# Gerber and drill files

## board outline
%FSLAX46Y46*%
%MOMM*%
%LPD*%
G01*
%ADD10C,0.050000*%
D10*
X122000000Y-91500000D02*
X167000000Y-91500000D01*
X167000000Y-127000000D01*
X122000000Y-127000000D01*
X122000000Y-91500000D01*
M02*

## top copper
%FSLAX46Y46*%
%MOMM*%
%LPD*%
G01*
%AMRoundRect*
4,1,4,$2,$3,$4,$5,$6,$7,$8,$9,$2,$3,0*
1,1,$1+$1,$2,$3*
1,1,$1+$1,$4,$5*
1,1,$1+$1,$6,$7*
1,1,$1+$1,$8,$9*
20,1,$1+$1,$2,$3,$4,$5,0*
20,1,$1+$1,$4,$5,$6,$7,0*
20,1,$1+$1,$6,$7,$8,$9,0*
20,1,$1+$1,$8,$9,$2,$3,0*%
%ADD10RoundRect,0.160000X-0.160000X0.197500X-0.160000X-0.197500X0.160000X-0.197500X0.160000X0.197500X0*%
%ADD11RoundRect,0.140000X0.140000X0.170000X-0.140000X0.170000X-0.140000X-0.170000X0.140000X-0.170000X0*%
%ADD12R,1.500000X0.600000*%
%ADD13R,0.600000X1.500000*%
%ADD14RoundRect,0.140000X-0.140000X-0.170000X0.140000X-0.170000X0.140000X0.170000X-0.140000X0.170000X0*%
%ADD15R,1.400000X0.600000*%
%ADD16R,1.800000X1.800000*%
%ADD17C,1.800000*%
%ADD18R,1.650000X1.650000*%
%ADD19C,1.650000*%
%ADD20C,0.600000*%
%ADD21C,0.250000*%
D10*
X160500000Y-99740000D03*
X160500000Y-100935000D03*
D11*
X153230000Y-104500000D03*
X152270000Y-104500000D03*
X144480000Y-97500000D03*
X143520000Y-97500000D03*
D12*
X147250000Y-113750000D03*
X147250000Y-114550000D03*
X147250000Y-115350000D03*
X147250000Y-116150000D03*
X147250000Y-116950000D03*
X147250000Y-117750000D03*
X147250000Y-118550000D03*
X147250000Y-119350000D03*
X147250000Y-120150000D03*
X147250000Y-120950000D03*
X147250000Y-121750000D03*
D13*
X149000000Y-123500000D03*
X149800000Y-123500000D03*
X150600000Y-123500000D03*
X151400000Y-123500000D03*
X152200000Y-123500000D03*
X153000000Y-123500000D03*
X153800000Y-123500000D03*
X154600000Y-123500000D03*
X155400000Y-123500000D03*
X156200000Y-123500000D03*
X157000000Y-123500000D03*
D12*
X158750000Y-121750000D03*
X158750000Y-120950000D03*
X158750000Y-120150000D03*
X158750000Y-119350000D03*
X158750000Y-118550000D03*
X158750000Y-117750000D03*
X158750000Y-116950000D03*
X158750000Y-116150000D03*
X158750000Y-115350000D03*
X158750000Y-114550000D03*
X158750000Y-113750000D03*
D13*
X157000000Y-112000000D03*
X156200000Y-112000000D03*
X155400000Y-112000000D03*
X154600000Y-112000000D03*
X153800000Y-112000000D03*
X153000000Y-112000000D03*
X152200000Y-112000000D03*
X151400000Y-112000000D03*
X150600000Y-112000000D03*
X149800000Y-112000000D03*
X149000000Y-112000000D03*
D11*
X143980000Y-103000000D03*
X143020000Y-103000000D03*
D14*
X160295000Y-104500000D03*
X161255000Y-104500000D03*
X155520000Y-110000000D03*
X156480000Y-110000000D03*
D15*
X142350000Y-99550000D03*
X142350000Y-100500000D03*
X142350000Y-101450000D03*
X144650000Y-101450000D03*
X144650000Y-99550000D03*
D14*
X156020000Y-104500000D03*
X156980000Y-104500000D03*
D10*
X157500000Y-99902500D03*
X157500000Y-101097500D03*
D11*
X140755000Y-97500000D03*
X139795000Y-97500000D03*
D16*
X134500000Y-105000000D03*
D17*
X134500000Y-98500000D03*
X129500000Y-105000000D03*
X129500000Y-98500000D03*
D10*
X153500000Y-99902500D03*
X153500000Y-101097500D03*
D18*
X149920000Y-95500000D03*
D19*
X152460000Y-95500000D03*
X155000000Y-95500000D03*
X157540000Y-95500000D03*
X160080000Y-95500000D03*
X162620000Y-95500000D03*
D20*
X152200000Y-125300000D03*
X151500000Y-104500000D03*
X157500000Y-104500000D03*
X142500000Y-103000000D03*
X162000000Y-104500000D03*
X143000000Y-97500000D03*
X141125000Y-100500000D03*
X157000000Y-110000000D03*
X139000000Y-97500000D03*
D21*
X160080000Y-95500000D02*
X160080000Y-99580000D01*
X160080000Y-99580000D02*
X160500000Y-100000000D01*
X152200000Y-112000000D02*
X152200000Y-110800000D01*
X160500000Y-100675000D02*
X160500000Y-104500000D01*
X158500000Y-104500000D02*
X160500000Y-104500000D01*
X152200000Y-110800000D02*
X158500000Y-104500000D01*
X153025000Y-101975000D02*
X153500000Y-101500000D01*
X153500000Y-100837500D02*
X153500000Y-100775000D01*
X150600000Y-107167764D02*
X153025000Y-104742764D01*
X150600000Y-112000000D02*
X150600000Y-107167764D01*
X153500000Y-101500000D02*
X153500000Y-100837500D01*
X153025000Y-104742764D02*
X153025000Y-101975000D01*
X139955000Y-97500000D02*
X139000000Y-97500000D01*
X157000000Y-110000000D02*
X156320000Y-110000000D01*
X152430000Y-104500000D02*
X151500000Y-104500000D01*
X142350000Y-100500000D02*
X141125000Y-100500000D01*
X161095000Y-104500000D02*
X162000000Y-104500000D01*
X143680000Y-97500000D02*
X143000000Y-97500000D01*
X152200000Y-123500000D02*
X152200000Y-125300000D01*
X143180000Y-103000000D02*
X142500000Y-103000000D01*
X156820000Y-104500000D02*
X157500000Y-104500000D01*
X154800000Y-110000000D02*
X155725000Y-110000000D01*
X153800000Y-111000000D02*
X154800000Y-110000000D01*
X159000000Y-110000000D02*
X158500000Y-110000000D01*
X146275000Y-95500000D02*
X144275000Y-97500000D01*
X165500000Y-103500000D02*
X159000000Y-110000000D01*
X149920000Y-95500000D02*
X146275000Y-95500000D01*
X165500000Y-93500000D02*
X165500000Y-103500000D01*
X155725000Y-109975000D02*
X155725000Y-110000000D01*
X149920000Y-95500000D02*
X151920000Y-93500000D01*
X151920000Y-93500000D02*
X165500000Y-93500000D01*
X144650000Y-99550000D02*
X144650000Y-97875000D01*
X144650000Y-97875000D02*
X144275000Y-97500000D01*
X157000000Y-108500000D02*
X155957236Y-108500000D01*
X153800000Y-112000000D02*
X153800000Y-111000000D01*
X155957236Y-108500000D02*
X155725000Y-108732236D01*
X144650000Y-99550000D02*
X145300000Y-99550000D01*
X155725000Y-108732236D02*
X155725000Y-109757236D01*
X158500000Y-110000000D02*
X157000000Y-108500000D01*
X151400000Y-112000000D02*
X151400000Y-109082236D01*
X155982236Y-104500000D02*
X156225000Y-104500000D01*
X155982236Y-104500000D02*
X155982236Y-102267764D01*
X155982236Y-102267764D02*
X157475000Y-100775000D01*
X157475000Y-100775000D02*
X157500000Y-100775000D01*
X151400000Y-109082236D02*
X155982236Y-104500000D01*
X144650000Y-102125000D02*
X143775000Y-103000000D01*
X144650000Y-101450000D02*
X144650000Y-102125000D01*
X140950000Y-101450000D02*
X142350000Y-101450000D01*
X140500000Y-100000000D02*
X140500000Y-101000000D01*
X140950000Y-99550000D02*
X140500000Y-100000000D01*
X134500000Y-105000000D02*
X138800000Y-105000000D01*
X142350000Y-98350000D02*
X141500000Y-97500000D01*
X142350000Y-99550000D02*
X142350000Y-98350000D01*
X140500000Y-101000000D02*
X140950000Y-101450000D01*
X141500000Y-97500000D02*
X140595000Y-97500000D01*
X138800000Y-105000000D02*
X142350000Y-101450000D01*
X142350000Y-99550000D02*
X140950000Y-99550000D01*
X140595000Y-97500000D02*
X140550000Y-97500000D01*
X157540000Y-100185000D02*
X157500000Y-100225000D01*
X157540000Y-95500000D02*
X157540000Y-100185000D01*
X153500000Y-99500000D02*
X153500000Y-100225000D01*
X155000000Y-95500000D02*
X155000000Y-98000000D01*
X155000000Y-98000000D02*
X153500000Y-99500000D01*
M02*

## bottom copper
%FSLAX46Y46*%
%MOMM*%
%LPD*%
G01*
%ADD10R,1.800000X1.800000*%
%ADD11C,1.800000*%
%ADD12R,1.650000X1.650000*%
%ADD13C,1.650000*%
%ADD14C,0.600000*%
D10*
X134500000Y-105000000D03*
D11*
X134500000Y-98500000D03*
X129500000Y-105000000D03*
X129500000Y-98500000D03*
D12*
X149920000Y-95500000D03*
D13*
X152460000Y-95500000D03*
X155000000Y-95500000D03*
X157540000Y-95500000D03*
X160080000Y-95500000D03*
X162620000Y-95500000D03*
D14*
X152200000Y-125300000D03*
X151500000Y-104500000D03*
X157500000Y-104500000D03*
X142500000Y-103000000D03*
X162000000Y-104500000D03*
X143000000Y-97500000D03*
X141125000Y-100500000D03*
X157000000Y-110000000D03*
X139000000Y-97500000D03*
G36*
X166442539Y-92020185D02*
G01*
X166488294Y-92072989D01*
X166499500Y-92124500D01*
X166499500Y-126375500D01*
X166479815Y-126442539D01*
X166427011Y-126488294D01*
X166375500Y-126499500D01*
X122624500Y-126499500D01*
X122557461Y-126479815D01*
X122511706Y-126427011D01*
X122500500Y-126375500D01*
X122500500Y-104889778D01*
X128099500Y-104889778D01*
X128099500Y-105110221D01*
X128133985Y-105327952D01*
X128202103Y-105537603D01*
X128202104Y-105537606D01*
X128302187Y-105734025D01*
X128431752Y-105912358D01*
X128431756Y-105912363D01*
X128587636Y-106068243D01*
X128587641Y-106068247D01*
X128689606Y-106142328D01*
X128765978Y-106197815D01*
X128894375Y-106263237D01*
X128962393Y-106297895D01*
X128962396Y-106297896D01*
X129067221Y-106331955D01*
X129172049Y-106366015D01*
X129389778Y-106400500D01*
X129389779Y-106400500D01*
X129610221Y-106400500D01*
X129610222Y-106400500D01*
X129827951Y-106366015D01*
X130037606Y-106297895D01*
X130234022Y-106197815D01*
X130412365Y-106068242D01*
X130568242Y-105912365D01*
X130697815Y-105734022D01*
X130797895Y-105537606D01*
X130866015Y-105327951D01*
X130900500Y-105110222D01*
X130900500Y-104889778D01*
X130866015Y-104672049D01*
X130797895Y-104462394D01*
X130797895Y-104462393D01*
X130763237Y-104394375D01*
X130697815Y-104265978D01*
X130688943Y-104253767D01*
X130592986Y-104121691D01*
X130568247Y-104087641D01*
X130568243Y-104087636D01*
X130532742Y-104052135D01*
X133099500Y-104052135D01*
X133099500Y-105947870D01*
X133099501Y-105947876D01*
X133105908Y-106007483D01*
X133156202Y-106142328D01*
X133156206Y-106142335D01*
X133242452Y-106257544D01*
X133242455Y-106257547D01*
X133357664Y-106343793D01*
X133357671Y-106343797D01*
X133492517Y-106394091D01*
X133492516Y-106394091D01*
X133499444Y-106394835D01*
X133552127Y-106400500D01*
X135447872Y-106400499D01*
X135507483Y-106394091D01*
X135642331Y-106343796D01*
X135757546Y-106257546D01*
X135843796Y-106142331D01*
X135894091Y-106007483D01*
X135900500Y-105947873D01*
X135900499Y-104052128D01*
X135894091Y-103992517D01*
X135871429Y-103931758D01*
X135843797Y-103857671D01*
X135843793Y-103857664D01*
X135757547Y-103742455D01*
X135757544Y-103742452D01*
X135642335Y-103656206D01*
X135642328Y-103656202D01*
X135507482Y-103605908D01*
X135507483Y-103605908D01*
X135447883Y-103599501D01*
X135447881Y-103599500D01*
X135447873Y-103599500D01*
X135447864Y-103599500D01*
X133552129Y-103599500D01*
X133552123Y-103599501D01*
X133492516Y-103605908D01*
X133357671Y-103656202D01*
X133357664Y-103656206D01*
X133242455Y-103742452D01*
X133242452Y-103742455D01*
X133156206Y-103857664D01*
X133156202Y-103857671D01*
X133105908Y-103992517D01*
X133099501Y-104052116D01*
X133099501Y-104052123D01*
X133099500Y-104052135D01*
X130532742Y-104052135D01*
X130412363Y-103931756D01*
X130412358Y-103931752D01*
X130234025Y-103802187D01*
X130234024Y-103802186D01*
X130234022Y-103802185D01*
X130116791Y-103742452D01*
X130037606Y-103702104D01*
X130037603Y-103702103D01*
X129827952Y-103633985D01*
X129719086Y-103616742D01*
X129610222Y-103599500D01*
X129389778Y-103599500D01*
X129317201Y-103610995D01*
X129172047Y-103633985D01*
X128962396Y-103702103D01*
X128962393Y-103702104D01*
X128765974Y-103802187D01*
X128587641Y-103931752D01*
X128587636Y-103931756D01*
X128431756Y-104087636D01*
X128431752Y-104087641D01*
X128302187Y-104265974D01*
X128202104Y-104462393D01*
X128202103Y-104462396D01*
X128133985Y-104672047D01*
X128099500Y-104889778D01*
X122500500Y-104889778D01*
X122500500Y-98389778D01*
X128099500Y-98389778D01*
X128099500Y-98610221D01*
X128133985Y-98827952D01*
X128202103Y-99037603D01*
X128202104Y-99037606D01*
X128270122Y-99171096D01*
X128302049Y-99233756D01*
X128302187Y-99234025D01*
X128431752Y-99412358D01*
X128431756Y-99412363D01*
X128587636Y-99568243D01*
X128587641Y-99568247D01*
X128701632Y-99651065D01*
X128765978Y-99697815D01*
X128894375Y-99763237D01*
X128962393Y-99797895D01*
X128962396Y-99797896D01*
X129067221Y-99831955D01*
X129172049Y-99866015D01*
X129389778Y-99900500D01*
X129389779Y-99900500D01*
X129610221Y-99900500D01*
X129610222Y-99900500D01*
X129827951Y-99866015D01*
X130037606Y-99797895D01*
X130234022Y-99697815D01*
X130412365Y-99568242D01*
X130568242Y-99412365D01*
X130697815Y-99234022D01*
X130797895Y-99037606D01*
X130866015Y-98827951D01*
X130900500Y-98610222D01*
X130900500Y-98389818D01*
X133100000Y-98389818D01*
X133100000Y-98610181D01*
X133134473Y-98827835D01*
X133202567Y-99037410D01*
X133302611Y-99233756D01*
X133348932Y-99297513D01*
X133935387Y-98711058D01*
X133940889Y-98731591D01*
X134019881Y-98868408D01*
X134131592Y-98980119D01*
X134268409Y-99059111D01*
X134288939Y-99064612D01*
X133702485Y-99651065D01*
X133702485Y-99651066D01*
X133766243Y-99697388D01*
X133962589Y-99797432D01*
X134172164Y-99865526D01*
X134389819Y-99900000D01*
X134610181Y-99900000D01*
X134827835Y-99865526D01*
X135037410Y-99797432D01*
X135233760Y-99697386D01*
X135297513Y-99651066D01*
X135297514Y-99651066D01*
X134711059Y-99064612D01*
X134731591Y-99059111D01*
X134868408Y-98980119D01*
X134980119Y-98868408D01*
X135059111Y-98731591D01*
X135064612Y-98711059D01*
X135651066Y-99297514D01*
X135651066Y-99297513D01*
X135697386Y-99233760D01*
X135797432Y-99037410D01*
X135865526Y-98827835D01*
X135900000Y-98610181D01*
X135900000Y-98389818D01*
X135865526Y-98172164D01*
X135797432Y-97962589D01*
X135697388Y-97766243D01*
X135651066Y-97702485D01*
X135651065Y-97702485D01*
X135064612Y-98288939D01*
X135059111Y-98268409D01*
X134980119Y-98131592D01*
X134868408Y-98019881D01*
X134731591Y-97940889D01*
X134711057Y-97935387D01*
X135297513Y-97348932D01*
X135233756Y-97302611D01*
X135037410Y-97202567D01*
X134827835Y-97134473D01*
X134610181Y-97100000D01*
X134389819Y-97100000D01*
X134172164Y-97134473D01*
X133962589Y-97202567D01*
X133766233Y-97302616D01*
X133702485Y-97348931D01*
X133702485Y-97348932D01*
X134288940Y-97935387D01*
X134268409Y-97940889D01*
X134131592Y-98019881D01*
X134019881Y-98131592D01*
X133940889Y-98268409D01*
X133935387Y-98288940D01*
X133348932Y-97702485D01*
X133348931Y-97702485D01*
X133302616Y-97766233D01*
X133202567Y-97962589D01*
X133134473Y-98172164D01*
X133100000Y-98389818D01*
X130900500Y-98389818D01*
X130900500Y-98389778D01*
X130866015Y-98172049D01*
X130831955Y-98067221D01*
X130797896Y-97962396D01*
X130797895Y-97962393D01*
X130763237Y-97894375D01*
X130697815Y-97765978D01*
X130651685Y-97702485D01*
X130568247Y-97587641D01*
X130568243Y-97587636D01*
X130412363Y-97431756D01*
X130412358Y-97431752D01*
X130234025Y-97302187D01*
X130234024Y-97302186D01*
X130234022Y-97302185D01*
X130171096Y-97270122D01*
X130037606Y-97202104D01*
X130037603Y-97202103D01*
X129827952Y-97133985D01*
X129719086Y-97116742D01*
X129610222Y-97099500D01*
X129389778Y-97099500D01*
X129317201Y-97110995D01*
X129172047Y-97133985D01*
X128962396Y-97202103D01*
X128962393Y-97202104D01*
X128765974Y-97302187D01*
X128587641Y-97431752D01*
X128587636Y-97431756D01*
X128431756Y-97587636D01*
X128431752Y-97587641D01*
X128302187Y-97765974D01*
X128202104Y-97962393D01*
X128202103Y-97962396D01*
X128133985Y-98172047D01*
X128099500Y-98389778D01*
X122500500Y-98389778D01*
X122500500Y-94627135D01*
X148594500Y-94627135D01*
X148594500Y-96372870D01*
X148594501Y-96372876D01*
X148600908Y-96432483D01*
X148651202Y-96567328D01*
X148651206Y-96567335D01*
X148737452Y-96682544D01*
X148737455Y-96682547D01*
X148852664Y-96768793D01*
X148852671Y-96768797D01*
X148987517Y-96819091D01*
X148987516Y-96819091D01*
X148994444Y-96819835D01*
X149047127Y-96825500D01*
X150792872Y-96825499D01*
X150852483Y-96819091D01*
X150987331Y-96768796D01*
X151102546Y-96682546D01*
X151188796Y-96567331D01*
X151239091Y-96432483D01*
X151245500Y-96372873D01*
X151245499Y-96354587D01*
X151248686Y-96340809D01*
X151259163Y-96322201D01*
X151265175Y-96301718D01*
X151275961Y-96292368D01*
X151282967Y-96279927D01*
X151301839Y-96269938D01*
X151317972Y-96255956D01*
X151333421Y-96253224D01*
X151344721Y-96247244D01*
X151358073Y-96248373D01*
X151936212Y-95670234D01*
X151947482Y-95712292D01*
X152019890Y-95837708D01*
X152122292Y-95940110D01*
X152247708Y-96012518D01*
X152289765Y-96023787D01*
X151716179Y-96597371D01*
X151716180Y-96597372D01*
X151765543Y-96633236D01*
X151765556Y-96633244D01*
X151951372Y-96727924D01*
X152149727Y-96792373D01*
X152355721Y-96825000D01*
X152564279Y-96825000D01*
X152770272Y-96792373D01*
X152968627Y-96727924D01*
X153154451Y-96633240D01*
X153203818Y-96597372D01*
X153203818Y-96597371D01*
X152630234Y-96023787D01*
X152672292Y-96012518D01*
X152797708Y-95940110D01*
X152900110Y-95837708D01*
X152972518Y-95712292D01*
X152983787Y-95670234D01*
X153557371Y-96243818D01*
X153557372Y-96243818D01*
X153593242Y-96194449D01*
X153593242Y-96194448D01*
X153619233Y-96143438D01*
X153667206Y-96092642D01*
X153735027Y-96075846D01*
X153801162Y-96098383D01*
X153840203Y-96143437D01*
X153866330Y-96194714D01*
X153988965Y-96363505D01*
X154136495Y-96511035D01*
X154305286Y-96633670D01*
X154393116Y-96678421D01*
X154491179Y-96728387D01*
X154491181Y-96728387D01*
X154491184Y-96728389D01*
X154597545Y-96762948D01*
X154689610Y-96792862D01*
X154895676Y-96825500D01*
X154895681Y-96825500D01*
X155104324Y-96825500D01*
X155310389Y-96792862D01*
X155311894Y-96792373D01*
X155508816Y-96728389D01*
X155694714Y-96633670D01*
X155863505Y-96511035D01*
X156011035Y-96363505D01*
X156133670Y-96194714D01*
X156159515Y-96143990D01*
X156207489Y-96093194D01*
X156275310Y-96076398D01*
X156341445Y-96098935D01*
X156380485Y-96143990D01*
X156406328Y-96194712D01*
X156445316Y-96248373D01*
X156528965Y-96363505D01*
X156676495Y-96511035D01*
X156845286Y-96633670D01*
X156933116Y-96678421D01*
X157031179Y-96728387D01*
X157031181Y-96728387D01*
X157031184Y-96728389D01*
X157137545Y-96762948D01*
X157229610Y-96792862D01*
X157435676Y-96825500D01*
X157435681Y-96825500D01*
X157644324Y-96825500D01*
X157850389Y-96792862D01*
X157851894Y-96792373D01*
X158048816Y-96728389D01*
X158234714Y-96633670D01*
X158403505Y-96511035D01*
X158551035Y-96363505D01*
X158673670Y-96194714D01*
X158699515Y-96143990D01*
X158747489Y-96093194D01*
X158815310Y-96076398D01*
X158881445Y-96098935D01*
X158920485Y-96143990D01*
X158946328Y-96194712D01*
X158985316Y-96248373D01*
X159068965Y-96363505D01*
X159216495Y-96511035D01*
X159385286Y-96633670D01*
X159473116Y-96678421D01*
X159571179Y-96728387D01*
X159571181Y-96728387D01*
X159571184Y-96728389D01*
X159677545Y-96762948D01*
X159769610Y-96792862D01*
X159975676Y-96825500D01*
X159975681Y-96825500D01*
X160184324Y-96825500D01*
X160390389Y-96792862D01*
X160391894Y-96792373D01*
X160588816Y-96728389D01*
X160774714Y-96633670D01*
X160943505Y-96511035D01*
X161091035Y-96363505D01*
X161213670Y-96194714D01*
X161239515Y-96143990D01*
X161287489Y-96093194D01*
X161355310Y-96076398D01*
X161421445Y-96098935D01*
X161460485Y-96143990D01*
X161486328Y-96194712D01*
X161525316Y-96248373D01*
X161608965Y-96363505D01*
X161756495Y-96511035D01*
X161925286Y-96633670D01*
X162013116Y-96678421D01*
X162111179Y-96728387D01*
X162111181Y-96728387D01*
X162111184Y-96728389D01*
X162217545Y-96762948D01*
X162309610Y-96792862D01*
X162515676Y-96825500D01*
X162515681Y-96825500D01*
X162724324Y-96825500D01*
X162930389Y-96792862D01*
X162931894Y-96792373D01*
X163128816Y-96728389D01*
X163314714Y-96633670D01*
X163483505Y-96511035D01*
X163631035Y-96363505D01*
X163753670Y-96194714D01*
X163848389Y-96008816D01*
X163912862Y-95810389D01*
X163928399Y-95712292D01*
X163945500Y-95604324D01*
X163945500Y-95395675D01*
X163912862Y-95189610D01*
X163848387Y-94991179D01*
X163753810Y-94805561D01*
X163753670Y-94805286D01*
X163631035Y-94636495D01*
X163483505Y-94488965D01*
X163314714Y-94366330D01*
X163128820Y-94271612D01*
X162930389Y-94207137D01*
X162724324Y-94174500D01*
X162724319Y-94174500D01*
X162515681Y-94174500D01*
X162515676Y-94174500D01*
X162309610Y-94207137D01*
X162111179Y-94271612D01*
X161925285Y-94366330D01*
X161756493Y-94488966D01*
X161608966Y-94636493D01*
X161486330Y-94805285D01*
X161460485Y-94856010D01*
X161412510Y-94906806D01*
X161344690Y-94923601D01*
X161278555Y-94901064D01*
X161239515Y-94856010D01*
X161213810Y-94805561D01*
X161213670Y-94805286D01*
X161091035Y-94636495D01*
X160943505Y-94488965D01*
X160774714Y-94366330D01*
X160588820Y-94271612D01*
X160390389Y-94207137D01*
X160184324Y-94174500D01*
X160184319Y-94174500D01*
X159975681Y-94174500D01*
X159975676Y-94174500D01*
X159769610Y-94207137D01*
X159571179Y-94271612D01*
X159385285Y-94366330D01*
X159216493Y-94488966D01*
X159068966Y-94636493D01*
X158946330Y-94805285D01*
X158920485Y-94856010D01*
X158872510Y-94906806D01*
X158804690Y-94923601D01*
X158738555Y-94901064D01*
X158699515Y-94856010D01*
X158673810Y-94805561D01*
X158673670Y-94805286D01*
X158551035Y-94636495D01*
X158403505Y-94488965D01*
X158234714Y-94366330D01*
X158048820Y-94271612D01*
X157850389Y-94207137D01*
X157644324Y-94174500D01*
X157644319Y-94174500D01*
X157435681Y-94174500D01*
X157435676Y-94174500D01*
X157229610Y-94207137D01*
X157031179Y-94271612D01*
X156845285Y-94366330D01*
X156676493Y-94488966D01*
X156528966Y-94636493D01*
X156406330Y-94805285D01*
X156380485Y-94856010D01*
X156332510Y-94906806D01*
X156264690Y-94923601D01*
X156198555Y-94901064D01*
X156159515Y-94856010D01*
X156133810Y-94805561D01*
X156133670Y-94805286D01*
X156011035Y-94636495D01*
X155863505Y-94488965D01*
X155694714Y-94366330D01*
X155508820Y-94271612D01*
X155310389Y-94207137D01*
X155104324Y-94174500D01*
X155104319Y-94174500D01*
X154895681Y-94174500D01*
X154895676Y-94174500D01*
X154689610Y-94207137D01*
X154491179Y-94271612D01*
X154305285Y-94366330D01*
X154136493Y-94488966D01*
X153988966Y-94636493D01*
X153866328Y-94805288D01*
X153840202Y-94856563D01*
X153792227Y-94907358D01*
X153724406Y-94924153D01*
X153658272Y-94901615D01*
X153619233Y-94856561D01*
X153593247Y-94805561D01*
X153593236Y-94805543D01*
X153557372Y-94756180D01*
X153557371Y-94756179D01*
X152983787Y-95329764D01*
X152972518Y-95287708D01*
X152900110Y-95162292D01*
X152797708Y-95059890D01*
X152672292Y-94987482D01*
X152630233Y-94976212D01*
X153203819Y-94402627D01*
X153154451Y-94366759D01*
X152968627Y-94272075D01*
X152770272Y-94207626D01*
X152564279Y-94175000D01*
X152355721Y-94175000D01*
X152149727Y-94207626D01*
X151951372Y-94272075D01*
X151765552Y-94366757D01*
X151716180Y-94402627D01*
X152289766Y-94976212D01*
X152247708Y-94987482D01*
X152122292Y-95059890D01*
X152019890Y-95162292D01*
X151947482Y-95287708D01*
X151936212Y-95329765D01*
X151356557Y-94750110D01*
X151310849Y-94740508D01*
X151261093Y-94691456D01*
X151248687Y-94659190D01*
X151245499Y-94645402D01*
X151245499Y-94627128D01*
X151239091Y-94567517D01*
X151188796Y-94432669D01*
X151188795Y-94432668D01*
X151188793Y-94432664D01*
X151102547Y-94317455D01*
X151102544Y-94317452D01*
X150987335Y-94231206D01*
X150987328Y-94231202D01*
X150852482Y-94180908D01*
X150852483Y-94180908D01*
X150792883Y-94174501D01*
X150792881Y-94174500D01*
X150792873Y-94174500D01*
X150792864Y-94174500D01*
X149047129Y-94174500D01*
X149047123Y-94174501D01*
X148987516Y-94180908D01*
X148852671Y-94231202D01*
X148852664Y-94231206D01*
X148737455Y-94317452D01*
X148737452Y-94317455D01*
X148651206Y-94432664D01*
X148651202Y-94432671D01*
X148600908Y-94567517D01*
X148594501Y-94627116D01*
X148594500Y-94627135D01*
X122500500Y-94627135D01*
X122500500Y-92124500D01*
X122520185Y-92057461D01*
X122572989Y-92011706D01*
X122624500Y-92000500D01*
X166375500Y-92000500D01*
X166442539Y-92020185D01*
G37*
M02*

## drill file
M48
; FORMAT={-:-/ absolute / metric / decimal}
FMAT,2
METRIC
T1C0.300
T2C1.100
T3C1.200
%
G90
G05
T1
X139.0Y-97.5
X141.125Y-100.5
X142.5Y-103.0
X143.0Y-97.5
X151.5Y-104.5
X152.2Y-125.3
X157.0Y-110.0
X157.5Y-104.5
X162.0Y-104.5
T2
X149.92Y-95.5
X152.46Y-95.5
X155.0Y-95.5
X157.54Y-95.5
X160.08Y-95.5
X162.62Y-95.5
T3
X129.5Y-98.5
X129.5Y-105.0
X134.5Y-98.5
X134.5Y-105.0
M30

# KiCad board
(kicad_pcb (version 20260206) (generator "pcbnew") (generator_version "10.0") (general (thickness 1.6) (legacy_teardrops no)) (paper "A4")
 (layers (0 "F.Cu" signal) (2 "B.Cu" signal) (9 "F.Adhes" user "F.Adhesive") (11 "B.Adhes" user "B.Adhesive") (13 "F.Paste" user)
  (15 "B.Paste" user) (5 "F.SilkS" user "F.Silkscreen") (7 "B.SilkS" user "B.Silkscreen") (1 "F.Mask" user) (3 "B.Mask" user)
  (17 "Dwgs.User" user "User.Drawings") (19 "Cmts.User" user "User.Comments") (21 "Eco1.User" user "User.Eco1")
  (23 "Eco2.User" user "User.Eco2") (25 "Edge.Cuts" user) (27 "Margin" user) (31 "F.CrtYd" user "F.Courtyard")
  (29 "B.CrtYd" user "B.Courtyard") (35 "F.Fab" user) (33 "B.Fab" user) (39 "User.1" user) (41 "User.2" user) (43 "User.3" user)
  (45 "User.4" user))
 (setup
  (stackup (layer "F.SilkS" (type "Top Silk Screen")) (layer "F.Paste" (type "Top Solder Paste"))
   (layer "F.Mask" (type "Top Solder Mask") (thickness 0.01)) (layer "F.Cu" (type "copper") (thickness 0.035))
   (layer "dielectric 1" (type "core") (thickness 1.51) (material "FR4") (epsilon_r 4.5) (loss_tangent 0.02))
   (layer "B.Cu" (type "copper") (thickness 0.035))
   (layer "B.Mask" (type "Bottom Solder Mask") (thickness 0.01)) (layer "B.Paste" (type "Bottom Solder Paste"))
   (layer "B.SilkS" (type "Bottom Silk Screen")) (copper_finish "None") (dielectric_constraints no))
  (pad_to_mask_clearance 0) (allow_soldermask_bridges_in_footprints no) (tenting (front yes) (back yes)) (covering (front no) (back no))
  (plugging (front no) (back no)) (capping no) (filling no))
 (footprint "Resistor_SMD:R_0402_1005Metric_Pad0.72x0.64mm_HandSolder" (layer "F.Cu") (at 160.5 100.3375 -90)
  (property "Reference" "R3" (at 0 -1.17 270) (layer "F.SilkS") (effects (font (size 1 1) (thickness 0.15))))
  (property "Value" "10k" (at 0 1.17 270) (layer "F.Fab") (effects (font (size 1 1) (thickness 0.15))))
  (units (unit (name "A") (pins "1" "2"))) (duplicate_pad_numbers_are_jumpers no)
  (pad "1" smd roundrect (at -0.5975 0 270) (size 0.715 0.64) (layers "F.Cu" "F.Mask" "F.Paste") (roundrect_rratio 0.25)
   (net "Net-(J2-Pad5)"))
  (pad "2" smd roundrect (at 0.5975 0 270) (size 0.715 0.64) (layers "F.Cu" "F.Mask" "F.Paste") (roundrect_rratio 0.25)
   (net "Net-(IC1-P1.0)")))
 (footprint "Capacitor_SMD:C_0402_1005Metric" (layer "F.Cu") (at 152.75 104.5 180)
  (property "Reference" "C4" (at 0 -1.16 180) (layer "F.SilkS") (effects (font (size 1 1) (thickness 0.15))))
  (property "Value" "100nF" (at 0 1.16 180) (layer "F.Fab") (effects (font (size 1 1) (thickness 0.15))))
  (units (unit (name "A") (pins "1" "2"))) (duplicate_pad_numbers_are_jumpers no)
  (pad "1" smd roundrect (at -0.48 0 180) (size 0.56 0.62) (layers "F.Cu" "F.Mask" "F.Paste") (roundrect_rratio 0.25) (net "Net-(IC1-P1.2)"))
  (pad "2" smd roundrect (at 0.48 0 180) (size 0.56 0.62) (layers "F.Cu" "F.Mask" "F.Paste") (roundrect_rratio 0.25) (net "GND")))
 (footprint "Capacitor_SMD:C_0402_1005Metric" (layer "F.Cu") (at 144 97.5 180)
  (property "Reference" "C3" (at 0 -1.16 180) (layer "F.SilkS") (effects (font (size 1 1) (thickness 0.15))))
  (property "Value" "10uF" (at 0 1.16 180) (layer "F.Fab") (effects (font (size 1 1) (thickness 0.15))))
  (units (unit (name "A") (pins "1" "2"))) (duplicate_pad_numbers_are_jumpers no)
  (pad "1" smd roundrect (at -0.48 0 180) (size 0.56 0.62) (layers "F.Cu" "F.Mask" "F.Paste") (roundrect_rratio 0.25)
   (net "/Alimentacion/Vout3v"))
  (pad "2" smd roundrect (at 0.48 0 180) (size 0.56 0.62) (layers "F.Cu" "F.Mask" "F.Paste") (roundrect_rratio 0.25) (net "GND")))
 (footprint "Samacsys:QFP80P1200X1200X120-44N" (layer "F.Cu") (at 153 117.75)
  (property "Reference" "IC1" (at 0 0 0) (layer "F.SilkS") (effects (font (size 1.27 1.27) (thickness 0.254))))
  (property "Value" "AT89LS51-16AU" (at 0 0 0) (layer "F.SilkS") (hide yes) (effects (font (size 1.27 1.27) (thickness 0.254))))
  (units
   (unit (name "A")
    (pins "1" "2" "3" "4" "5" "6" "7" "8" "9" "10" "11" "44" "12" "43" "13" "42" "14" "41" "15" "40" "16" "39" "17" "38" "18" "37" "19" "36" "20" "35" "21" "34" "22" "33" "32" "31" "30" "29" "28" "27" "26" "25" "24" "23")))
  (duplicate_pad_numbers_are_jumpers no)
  (pad "1" smd rect (at -5.75 -4 90) (size 0.6 1.5) (layers "F.Cu" "F.Mask" "F.Paste") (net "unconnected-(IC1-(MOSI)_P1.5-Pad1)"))
  (pad "2" smd rect (at -5.75 -3.2 90) (size 0.6 1.5) (layers "F.Cu" "F.Mask" "F.Paste") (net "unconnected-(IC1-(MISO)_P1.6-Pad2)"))
  (pad "3" smd rect (at -5.75 -2.4 90) (size 0.6 1.5) (layers "F.Cu" "F.Mask" "F.Paste") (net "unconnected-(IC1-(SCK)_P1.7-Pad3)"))
  (pad "4" smd rect (at -5.75 -1.6 90) (size 0.6 1.5) (layers "F.Cu" "F.Mask" "F.Paste") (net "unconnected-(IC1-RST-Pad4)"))
  (pad "5" smd rect (at -5.75 -0.8 90) (size 0.6 1.5) (layers "F.Cu" "F.Mask" "F.Paste") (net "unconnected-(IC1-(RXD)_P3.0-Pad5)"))
  (pad "6" smd rect (at -5.75 0 90) (size 0.6 1.5) (layers "F.Cu" "F.Mask" "F.Paste") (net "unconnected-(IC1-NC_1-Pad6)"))
  (pad "7" smd rect (at -5.75 0.8 90) (size 0.6 1.5) (layers "F.Cu" "F.Mask" "F.Paste") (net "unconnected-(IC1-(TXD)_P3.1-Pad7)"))
  (pad "8" smd rect (at -5.75 1.6 90) (size 0.6 1.5) (layers "F.Cu" "F.Mask" "F.Paste") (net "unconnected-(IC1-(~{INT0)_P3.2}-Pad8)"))
  (pad "9" smd rect (at -5.75 2.4 90) (size 0.6 1.5) (layers "F.Cu" "F.Mask" "F.Paste") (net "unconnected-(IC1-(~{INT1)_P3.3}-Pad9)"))
  (pad "10" smd rect (at -5.75 3.2 90) (size 0.6 1.5) (layers "F.Cu" "F.Mask" "F.Paste") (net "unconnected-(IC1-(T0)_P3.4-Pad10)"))
  (pad "11" smd rect (at -5.75 4 90) (size 0.6 1.5) (layers "F.Cu" "F.Mask" "F.Paste") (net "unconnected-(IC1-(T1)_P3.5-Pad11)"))
  (pad "12" smd rect (at -4 5.75) (size 0.6 1.5) (layers "F.Cu" "F.Mask" "F.Paste") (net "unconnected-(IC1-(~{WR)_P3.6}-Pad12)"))
  (pad "13" smd rect (at -3.2 5.75) (size 0.6 1.5) (layers "F.Cu" "F.Mask" "F.Paste") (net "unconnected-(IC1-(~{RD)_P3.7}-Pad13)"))
  (pad "14" smd rect (at -2.4 5.75) (size 0.6 1.5) (layers "F.Cu" "F.Mask" "F.Paste") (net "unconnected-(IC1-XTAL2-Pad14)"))
  (pad "15" smd rect (at -1.6 5.75) (size 0.6 1.5) (layers "F.Cu" "F.Mask" "F.Paste") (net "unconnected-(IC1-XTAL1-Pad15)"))
  (pad "16" smd rect (at -0.8 5.75) (size 0.6 1.5) (layers "F.Cu" "F.Mask" "F.Paste") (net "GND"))
  (pad "17" smd rect (at 0 5.75) (size 0.6 1.5) (layers "F.Cu" "F.Mask" "F.Paste") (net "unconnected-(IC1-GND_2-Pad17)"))
  (pad "18" smd rect (at 0.8 5.75) (size 0.6 1.5) (layers "F.Cu" "F.Mask" "F.Paste") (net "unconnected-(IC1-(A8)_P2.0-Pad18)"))
  (pad "19" smd rect (at 1.6 5.75) (size 0.6 1.5) (layers "F.Cu" "F.Mask" "F.Paste") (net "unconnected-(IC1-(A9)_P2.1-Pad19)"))
  (pad "20" smd rect (at 2.4 5.75) (size 0.6 1.5) (layers "F.Cu" "F.Mask" "F.Paste") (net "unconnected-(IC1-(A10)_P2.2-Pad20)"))
  (pad "21" smd rect (at 3.2 5.75) (size 0.6 1.5) (layers "F.Cu" "F.Mask" "F.Paste") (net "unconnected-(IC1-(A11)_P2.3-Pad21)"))
  (pad "22" smd rect (at 4 5.75) (size 0.6 1.5) (layers "F.Cu" "F.Mask" "F.Paste") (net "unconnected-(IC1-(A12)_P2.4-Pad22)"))
  (pad "23" smd rect (at 5.75 4 90) (size 0.6 1.5) (layers "F.Cu" "F.Mask" "F.Paste") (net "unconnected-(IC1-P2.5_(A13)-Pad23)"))
  (pad "24" smd rect (at 5.75 3.2 90) (size 0.6 1.5) (layers "F.Cu" "F.Mask" "F.Paste") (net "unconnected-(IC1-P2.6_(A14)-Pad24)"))
  (pad "25" smd rect (at 5.75 2.4 90) (size 0.6 1.5) (layers "F.Cu" "F.Mask" "F.Paste") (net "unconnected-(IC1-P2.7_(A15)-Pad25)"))
  (pad "26" smd rect (at 5.75 1.6 90) (size 0.6 1.5) (layers "F.Cu" "F.Mask" "F.Paste") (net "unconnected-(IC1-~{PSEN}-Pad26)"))
  (pad "27" smd rect (at 5.75 0.8 90) (size 0.6 1.5) (layers "F.Cu" "F.Mask" "F.Paste") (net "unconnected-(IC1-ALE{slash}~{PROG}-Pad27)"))
  (pad "28" smd rect (at 5.75 0 90) (size 0.6 1.5) (layers "F.Cu" "F.Mask" "F.Paste") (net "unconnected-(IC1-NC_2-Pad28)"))
  (pad "29" smd rect (at 5.75 -0.8 90) (size 0.6 1.5) (layers "F.Cu" "F.Mask" "F.Paste") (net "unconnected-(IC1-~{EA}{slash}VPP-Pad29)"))
  (pad "30" smd rect (at 5.75 -1.6 90) (size 0.6 1.5) (layers "F.Cu" "F.Mask" "F.Paste") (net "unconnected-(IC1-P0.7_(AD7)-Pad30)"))
  (pad "31" smd rect (at 5.75 -2.4 90) (size 0.6 1.5) (layers "F.Cu" "F.Mask" "F.Paste") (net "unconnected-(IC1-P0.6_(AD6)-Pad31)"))
  (pad "32" smd rect (at 5.75 -3.2 90) (size 0.6 1.5) (layers "F.Cu" "F.Mask" "F.Paste") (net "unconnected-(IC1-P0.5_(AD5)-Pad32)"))
  (pad "33" smd rect (at 5.75 -4 90) (size 0.6 1.5) (layers "F.Cu" "F.Mask" "F.Paste") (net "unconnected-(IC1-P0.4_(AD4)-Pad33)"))
  (pad "34" smd rect (at 4 -5.75) (size 0.6 1.5) (layers "F.Cu" "F.Mask" "F.Paste") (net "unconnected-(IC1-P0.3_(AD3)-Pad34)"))
  (pad "35" smd rect (at 3.2 -5.75) (size 0.6 1.5) (layers "F.Cu" "F.Mask" "F.Paste") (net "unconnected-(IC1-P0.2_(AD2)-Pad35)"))
  (pad "36" smd rect (at 2.4 -5.75) (size 0.6 1.5) (layers "F.Cu" "F.Mask" "F.Paste") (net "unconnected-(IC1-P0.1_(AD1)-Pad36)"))
  (pad "37" smd rect (at 1.6 -5.75) (size 0.6 1.5) (layers "F.Cu" "F.Mask" "F.Paste") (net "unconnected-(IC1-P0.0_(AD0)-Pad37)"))
  (pad "38" smd rect (at 0.8 -5.75) (size 0.6 1.5) (layers "F.Cu" "F.Mask" "F.Paste") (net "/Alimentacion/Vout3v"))
  (pad "39" smd rect (at 0 -5.75) (size 0.6 1.5) (layers "F.Cu" "F.Mask" "F.Paste") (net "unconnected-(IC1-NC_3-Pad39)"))
  (pad "40" smd rect (at -0.8 -5.75) (size 0.6 1.5) (layers "F.Cu" "F.Mask" "F.Paste") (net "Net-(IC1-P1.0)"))
  (pad "41" smd rect (at -1.6 -5.75) (size 0.6 1.5) (layers "F.Cu" "F.Mask" "F.Paste") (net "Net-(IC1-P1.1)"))
  (pad "42" smd rect (at -2.4 -5.75) (size 0.6 1.5) (layers "F.Cu" "F.Mask" "F.Paste") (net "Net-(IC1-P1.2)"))
  (pad "43" smd rect (at -3.2 -5.75) (size 0.6 1.5) (layers "F.Cu" "F.Mask" "F.Paste") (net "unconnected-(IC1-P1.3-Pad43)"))
  (pad "44" smd rect (at -4 -5.75) (size 0.6 1.5) (layers "F.Cu" "F.Mask" "F.Paste") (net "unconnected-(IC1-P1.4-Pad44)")))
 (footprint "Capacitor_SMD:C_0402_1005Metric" (layer "F.Cu") (at 143.5 103 180)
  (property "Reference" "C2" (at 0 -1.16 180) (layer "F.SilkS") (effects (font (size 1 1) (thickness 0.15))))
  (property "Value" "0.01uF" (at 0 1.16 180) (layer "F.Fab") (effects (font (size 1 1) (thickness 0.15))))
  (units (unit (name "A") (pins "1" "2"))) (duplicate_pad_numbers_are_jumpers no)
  (pad "1" smd roundrect (at -0.48 0 180) (size 0.56 0.62) (layers "F.Cu" "F.Mask" "F.Paste") (roundrect_rratio 0.25)
   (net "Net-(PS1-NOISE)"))
  (pad "2" smd roundrect (at 0.48 0 180) (size 0.56 0.62) (layers "F.Cu" "F.Mask" "F.Paste") (roundrect_rratio 0.25) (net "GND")))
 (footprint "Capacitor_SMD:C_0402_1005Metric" (layer "F.Cu") (at 160.775 104.5)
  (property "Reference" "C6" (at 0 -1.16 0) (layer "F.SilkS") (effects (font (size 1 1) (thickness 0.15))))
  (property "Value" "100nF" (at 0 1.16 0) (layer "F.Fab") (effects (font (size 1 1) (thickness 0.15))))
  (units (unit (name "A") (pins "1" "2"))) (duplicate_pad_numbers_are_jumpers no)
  (pad "1" smd roundrect (at -0.48 0) (size 0.56 0.62) (layers "F.Cu" "F.Mask" "F.Paste") (roundrect_rratio 0.25) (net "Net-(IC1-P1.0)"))
  (pad "2" smd roundrect (at 0.48 0) (size 0.56 0.62) (layers "F.Cu" "F.Mask" "F.Paste") (roundrect_rratio 0.25) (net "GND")))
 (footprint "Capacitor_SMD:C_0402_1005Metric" (layer "F.Cu") (at 156 110)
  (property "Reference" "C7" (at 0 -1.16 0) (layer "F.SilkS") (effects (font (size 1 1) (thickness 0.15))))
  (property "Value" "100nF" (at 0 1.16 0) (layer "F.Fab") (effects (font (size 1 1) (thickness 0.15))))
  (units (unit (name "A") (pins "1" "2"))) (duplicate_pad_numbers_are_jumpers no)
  (pad "1" smd roundrect (at -0.48 0) (size 0.56 0.62) (layers "F.Cu" "F.Mask" "F.Paste") (roundrect_rratio 0.25)
   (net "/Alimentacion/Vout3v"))
  (pad "2" smd roundrect (at 0.48 0) (size 0.56 0.62) (layers "F.Cu" "F.Mask" "F.Paste") (roundrect_rratio 0.25) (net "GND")))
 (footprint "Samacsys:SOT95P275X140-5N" (layer "F.Cu") (at 143.5 100.5)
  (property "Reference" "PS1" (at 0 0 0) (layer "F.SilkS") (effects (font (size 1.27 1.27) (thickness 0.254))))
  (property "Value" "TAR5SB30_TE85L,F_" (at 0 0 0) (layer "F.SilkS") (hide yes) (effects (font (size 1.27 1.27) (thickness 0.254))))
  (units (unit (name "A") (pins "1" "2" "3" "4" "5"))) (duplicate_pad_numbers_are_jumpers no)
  (pad "1" smd rect (at -1.15 -0.95 90) (size 0.6 1.4) (layers "F.Cu" "F.Mask" "F.Paste") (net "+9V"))
  (pad "2" smd rect (at -1.15 0 90) (size 0.6 1.4) (layers "F.Cu" "F.Mask" "F.Paste") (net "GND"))
  (pad "3" smd rect (at -1.15 0.95 90) (size 0.6 1.4) (layers "F.Cu" "F.Mask" "F.Paste") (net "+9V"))
  (pad "4" smd rect (at 1.15 0.95 90) (size 0.6 1.4) (layers "F.Cu" "F.Mask" "F.Paste") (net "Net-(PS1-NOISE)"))
  (pad "5" smd rect (at 1.15 -0.95 90) (size 0.6 1.4) (layers "F.Cu" "F.Mask" "F.Paste") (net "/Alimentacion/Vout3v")))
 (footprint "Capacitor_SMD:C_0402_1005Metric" (layer "F.Cu") (at 156.5 104.5)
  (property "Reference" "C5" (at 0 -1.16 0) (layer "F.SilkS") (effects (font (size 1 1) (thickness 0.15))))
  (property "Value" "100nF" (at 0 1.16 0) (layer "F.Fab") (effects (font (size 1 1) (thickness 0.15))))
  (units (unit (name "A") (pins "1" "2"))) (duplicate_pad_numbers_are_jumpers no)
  (pad "1" smd roundrect (at -0.48 0) (size 0.56 0.62) (layers "F.Cu" "F.Mask" "F.Paste") (roundrect_rratio 0.25) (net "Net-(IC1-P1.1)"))
  (pad "2" smd roundrect (at 0.48 0) (size 0.56 0.62) (layers "F.Cu" "F.Mask" "F.Paste") (roundrect_rratio 0.25) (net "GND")))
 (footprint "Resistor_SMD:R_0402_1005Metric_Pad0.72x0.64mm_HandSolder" (layer "F.Cu") (at 157.5 100.5 -90)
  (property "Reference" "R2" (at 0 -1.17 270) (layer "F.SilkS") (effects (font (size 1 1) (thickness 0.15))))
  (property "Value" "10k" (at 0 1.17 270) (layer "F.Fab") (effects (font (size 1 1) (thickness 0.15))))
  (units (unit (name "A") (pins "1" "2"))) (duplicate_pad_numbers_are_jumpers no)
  (pad "1" smd roundrect (at -0.5975 0 270) (size 0.715 0.64) (layers "F.Cu" "F.Mask" "F.Paste") (roundrect_rratio 0.25)
   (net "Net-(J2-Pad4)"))
  (pad "2" smd roundrect (at 0.5975 0 270) (size 0.715 0.64) (layers "F.Cu" "F.Mask" "F.Paste") (roundrect_rratio 0.25)
   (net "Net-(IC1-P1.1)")))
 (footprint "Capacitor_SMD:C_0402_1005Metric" (layer "F.Cu") (at 140.275 97.5 180)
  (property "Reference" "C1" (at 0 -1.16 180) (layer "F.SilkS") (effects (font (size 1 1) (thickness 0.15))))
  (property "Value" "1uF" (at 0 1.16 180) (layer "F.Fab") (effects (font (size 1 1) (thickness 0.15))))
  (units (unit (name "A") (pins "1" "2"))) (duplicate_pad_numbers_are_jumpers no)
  (pad "1" smd roundrect (at -0.48 0 180) (size 0.56 0.62) (layers "F.Cu" "F.Mask" "F.Paste") (roundrect_rratio 0.25) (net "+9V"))
  (pad "2" smd roundrect (at 0.48 0 180) (size 0.56 0.62) (layers "F.Cu" "F.Mask" "F.Paste") (roundrect_rratio 0.25) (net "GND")))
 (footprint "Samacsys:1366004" (layer "F.Cu") (at 134.5 105 180)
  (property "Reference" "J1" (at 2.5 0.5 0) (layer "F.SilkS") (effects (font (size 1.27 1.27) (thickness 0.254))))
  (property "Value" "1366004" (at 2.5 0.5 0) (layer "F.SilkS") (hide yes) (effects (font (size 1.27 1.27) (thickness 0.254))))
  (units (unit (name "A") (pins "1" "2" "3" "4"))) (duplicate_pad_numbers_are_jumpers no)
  (pad "1" thru_hole rect (at 0 0 180) (size 1.8 1.8) (drill 1.2) (layers "*.Cu" "*.Mask") (remove_unused_layers no) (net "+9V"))
  (pad "2" thru_hole circle (at 0 6.5 180) (size 1.8 1.8) (drill 1.2) (layers "*.Cu" "*.Mask") (remove_unused_layers no) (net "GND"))
  (pad "3" thru_hole circle (at 5 0 180) (size 1.8 1.8) (drill 1.2) (layers "*.Cu" "*.Mask") (remove_unused_layers no)
   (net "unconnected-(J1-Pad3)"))
  (pad "4" thru_hole circle (at 5 6.5 180) (size 1.8 1.8) (drill 1.2) (layers "*.Cu" "*.Mask") (remove_unused_layers no)
   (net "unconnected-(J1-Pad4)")))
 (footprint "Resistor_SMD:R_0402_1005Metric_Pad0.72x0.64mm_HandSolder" (layer "F.Cu") (at 153.5 100.5 -90)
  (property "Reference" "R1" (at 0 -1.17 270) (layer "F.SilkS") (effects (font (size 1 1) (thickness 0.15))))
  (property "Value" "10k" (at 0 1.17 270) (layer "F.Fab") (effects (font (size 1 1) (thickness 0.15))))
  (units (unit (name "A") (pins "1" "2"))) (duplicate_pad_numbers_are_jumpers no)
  (pad "1" smd roundrect (at -0.5975 0 270) (size 0.715 0.64) (layers "F.Cu" "F.Mask" "F.Paste") (roundrect_rratio 0.25)
   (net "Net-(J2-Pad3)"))
  (pad "2" smd roundrect (at 0.5975 0 270) (size 0.715 0.64) (layers "F.Cu" "F.Mask" "F.Paste") (roundrect_rratio 0.25)
   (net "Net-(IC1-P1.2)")))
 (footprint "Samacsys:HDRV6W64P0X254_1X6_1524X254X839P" (layer "F.Cu") (at 149.92 95.5)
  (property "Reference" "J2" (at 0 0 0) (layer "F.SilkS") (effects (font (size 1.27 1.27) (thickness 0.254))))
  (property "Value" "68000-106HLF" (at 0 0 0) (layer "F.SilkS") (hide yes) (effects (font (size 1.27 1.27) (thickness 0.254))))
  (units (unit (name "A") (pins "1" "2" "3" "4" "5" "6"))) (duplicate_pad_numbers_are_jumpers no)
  (pad "1" thru_hole rect (at 0 0) (size 1.65 1.65) (drill 1.1) (layers "*.Cu" "*.Mask") (remove_unused_layers no)
   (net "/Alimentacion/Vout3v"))
  (pad "2" thru_hole circle (at 2.54 0) (size 1.65 1.65) (drill 1.1) (layers "*.Cu" "*.Mask") (remove_unused_layers no) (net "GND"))
  (pad "3" thru_hole circle (at 5.08 0) (size 1.65 1.65) (drill 1.1) (layers "*.Cu" "*.Mask") (remove_unused_layers no)
   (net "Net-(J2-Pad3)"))
  (pad "4" thru_hole circle (at 7.62 0) (size 1.65 1.65) (drill 1.1) (layers "*.Cu" "*.Mask") (remove_unused_layers no)
   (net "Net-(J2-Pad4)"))
  (pad "5" thru_hole circle (at 10.16 0) (size 1.65 1.65) (drill 1.1) (layers "*.Cu" "*.Mask") (remove_unused_layers no)
   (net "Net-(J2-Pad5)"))
  (pad "6" thru_hole circle (at 12.7 0) (size 1.65 1.65) (drill 1.1) (layers "*.Cu" "*.Mask") (remove_unused_layers no)
   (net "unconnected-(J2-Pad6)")))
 (gr_rect (start 122 91.5) (end 167 127) (stroke (width 0.05) (type default)) (fill no) (layer "Edge.Cuts"))
 (segment (start 160.08 95.5) (end 160.08 99.58) (width 0.25) (layer "F.Cu") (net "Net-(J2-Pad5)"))
 (segment (start 160.08 99.58) (end 160.5 100) (width 0.25) (layer "F.Cu") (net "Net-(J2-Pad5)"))
 (segment (start 152.2 112) (end 152.2 110.8) (width 0.25) (layer "F.Cu") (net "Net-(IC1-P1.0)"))
 (segment (start 160.5 100.675) (end 160.5 104.5) (width 0.25) (layer "F.Cu") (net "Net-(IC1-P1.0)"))
 (segment (start 158.5 104.5) (end 160.5 104.5) (width 0.25) (layer "F.Cu") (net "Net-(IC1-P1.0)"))
 (segment (start 152.2 110.8) (end 158.5 104.5) (width 0.25) (layer "F.Cu") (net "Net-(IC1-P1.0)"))
 (segment (start 153.025 101.975) (end 153.5 101.5) (width 0.25) (layer "F.Cu") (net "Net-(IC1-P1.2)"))
 (segment (start 153.5 100.8375) (end 153.5 100.775) (width 0.25) (layer "F.Cu") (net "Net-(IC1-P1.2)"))
 (segment (start 150.6 107.167764) (end 153.025 104.742764) (width 0.25) (layer "F.Cu") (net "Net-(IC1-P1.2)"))
 (segment (start 150.6 112) (end 150.6 107.167764) (width 0.25) (layer "F.Cu") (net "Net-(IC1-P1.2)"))
 (segment (start 153.5 101.5) (end 153.5 100.8375) (width 0.25) (layer "F.Cu") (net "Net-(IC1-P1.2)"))
 (segment (start 153.025 104.742764) (end 153.025 101.975) (width 0.25) (layer "F.Cu") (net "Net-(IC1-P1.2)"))
 (segment (start 139.955 97.5) (end 139 97.5) (width 0.25) (layer "F.Cu") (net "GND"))
 (segment (start 157 110) (end 156.32 110) (width 0.25) (layer "F.Cu") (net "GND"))
 (segment (start 152.43 104.5) (end 151.5 104.5) (width 0.25) (layer "F.Cu") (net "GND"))
 (segment (start 142.35 100.5) (end 141.125 100.5) (width 0.25) (layer "F.Cu") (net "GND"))
 (segment (start 161.095 104.5) (end 162 104.5) (width 0.25) (layer "F.Cu") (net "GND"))
 (segment (start 143.68 97.5) (end 143 97.5) (width 0.25) (layer "F.Cu") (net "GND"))
 (segment (start 152.2 123.5) (end 152.2 125.3) (width 0.25) (layer "F.Cu") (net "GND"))
 (segment (start 143.18 103) (end 142.5 103) (width 0.25) (layer "F.Cu") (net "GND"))
 (segment (start 156.82 104.5) (end 157.5 104.5) (width 0.25) (layer "F.Cu") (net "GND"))
 (via (at 152.2 125.3) (size 0.6) (drill 0.3) (layers "F.Cu" "B.Cu") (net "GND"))
 (via (at 151.5 104.5) (size 0.6) (drill 0.3) (layers "F.Cu" "B.Cu") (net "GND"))
 (via (at 157.5 104.5) (size 0.6) (drill 0.3) (layers "F.Cu" "B.Cu") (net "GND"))
 (via (at 142.5 103) (size 0.6) (drill 0.3) (layers "F.Cu" "B.Cu") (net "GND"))
 (via (at 162 104.5) (size 0.6) (drill 0.3) (layers "F.Cu" "B.Cu") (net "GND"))
 (via (at 143 97.5) (size 0.6) (drill 0.3) (layers "F.Cu" "B.Cu") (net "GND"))
 (via (at 141.125 100.5) (size 0.6) (drill 0.3) (layers "F.Cu" "B.Cu") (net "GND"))
 (via (at 157 110) (size 0.6) (drill 0.3) (layers "F.Cu" "B.Cu") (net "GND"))
 (via (at 139 97.5) (size 0.6) (drill 0.3) (layers "F.Cu" "B.Cu") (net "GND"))
 (segment (start 154.8 110) (end 155.725 110) (width 0.25) (layer "F.Cu") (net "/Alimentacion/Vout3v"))
 (segment (start 153.8 111) (end 154.8 110) (width 0.25) (layer "F.Cu") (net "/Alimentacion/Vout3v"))
 (segment (start 159 110) (end 158.5 110) (width 0.25) (layer "F.Cu") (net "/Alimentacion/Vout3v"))
 (segment (start 146.275 95.5) (end 144.275 97.5) (width 0.25) (layer "F.Cu") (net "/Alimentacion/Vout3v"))
 (segment (start 165.5 103.5) (end 159 110) (width 0.25) (layer "F.Cu") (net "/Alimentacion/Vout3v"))
 (segment (start 149.92 95.5) (end 146.275 95.5) (width 0.25) (layer "F.Cu") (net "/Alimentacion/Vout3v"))
 (segment (start 165.5 93.5) (end 165.5 103.5) (width 0.25) (layer "F.Cu") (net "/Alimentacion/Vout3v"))
 (segment (start 155.725 109.975) (end 155.725 110) (width 0.25) (layer "F.Cu") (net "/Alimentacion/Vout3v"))
 (segment (start 149.92 95.5) (end 151.92 93.5) (width 0.25) (layer "F.Cu") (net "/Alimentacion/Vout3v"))
 (segment (start 151.92 93.5) (end 165.5 93.5) (width 0.25) (layer "F.Cu") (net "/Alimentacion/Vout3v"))
 (segment (start 144.65 99.55) (end 144.65 97.875) (width 0.25) (layer "F.Cu") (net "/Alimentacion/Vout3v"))
 (segment (start 144.65 97.875) (end 144.275 97.5) (width 0.25) (layer "F.Cu") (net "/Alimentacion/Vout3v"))
 (segment (start 157 108.5) (end 155.957236 108.5) (width 0.25) (layer "F.Cu") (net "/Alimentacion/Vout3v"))
 (segment (start 153.8 112) (end 153.8 111) (width 0.25) (layer "F.Cu") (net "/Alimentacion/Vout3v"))
 (segment (start 155.957236 108.5) (end 155.725 108.732236) (width 0.25) (layer "F.Cu") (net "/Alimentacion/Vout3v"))
 (segment (start 144.65 99.55) (end 145.3 99.55) (width 0.25) (layer "F.Cu") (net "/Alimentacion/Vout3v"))
 (segment (start 155.725 108.732236) (end 155.725 109.757236) (width 0.25) (layer "F.Cu") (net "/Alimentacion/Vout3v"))
 (segment (start 158.5 110) (end 157 108.5) (width 0.25) (layer "F.Cu") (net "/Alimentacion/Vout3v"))
 (segment (start 151.4 112) (end 151.4 109.082236) (width 0.25) (layer "F.Cu") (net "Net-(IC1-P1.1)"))
 (segment (start 155.982236 104.5) (end 156.225 104.5) (width 0.25) (layer "F.Cu") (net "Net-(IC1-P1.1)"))
 (segment (start 155.982236 104.5) (end 155.982236 102.267764) (width 0.25) (layer "F.Cu") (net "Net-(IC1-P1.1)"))
 (segment (start 155.982236 102.267764) (end 157.475 100.775) (width 0.25) (layer "F.Cu") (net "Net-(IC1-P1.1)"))
 (segment (start 157.475 100.775) (end 157.5 100.775) (width 0.25) (layer "F.Cu") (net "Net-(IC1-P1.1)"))
 (segment (start 151.4 109.082236) (end 155.982236 104.5) (width 0.25) (layer "F.Cu") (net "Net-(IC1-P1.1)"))
 (segment (start 144.65 102.125) (end 143.775 103) (width 0.25) (layer "F.Cu") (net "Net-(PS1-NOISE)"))
 (segment (start 144.65 101.45) (end 144.65 102.125) (width 0.25) (layer "F.Cu") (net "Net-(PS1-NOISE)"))
 (segment (start 140.95 101.45) (end 142.35 101.45) (width 0.25) (layer "F.Cu") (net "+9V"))
 (segment (start 140.5 100) (end 140.5 101) (width 0.25) (layer "F.Cu") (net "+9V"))
 (segment (start 140.95 99.55) (end 140.5 100) (width 0.25) (layer "F.Cu") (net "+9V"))
 (segment (start 134.5 105) (end 138.8 105) (width 0.25) (layer "F.Cu") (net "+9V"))
 (segment (start 142.35 98.35) (end 141.5 97.5) (width 0.25) (layer "F.Cu") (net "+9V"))
 (segment (start 142.35 99.55) (end 142.35 98.35) (width 0.25) (layer "F.Cu") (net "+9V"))
 (segment (start 140.5 101) (end 140.95 101.45) (width 0.25) (layer "F.Cu") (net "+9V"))
 (segment (start 141.5 97.5) (end 140.595 97.5) (width 0.25) (layer "F.Cu") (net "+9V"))
 (segment (start 138.8 105) (end 142.35 101.45) (width 0.25) (layer "F.Cu") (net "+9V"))
 (segment (start 142.35 99.55) (end 140.95 99.55) (width 0.25) (layer "F.Cu") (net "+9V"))
 (segment (start 140.595 97.5) (end 140.55 97.5) (width 0.25) (layer "F.Cu") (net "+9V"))
 (segment (start 157.54 100.185) (end 157.5 100.225) (width 0.25) (layer "F.Cu") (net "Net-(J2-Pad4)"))
 (segment (start 157.54 95.5) (end 157.54 100.185) (width 0.25) (layer "F.Cu") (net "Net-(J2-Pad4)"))
 (segment (start 153.5 99.5) (end 153.5 100.225) (width 0.25) (layer "F.Cu") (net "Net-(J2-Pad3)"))
 (segment (start 155 95.5) (end 155 98) (width 0.25) (layer "F.Cu") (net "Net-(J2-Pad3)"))
 (segment (start 155 98) (end 153.5 99.5) (width 0.25) (layer "F.Cu") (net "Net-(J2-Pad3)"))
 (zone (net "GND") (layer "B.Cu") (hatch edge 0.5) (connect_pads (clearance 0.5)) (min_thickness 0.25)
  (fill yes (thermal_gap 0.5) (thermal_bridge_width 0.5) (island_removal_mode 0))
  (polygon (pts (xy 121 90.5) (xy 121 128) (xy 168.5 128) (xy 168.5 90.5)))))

